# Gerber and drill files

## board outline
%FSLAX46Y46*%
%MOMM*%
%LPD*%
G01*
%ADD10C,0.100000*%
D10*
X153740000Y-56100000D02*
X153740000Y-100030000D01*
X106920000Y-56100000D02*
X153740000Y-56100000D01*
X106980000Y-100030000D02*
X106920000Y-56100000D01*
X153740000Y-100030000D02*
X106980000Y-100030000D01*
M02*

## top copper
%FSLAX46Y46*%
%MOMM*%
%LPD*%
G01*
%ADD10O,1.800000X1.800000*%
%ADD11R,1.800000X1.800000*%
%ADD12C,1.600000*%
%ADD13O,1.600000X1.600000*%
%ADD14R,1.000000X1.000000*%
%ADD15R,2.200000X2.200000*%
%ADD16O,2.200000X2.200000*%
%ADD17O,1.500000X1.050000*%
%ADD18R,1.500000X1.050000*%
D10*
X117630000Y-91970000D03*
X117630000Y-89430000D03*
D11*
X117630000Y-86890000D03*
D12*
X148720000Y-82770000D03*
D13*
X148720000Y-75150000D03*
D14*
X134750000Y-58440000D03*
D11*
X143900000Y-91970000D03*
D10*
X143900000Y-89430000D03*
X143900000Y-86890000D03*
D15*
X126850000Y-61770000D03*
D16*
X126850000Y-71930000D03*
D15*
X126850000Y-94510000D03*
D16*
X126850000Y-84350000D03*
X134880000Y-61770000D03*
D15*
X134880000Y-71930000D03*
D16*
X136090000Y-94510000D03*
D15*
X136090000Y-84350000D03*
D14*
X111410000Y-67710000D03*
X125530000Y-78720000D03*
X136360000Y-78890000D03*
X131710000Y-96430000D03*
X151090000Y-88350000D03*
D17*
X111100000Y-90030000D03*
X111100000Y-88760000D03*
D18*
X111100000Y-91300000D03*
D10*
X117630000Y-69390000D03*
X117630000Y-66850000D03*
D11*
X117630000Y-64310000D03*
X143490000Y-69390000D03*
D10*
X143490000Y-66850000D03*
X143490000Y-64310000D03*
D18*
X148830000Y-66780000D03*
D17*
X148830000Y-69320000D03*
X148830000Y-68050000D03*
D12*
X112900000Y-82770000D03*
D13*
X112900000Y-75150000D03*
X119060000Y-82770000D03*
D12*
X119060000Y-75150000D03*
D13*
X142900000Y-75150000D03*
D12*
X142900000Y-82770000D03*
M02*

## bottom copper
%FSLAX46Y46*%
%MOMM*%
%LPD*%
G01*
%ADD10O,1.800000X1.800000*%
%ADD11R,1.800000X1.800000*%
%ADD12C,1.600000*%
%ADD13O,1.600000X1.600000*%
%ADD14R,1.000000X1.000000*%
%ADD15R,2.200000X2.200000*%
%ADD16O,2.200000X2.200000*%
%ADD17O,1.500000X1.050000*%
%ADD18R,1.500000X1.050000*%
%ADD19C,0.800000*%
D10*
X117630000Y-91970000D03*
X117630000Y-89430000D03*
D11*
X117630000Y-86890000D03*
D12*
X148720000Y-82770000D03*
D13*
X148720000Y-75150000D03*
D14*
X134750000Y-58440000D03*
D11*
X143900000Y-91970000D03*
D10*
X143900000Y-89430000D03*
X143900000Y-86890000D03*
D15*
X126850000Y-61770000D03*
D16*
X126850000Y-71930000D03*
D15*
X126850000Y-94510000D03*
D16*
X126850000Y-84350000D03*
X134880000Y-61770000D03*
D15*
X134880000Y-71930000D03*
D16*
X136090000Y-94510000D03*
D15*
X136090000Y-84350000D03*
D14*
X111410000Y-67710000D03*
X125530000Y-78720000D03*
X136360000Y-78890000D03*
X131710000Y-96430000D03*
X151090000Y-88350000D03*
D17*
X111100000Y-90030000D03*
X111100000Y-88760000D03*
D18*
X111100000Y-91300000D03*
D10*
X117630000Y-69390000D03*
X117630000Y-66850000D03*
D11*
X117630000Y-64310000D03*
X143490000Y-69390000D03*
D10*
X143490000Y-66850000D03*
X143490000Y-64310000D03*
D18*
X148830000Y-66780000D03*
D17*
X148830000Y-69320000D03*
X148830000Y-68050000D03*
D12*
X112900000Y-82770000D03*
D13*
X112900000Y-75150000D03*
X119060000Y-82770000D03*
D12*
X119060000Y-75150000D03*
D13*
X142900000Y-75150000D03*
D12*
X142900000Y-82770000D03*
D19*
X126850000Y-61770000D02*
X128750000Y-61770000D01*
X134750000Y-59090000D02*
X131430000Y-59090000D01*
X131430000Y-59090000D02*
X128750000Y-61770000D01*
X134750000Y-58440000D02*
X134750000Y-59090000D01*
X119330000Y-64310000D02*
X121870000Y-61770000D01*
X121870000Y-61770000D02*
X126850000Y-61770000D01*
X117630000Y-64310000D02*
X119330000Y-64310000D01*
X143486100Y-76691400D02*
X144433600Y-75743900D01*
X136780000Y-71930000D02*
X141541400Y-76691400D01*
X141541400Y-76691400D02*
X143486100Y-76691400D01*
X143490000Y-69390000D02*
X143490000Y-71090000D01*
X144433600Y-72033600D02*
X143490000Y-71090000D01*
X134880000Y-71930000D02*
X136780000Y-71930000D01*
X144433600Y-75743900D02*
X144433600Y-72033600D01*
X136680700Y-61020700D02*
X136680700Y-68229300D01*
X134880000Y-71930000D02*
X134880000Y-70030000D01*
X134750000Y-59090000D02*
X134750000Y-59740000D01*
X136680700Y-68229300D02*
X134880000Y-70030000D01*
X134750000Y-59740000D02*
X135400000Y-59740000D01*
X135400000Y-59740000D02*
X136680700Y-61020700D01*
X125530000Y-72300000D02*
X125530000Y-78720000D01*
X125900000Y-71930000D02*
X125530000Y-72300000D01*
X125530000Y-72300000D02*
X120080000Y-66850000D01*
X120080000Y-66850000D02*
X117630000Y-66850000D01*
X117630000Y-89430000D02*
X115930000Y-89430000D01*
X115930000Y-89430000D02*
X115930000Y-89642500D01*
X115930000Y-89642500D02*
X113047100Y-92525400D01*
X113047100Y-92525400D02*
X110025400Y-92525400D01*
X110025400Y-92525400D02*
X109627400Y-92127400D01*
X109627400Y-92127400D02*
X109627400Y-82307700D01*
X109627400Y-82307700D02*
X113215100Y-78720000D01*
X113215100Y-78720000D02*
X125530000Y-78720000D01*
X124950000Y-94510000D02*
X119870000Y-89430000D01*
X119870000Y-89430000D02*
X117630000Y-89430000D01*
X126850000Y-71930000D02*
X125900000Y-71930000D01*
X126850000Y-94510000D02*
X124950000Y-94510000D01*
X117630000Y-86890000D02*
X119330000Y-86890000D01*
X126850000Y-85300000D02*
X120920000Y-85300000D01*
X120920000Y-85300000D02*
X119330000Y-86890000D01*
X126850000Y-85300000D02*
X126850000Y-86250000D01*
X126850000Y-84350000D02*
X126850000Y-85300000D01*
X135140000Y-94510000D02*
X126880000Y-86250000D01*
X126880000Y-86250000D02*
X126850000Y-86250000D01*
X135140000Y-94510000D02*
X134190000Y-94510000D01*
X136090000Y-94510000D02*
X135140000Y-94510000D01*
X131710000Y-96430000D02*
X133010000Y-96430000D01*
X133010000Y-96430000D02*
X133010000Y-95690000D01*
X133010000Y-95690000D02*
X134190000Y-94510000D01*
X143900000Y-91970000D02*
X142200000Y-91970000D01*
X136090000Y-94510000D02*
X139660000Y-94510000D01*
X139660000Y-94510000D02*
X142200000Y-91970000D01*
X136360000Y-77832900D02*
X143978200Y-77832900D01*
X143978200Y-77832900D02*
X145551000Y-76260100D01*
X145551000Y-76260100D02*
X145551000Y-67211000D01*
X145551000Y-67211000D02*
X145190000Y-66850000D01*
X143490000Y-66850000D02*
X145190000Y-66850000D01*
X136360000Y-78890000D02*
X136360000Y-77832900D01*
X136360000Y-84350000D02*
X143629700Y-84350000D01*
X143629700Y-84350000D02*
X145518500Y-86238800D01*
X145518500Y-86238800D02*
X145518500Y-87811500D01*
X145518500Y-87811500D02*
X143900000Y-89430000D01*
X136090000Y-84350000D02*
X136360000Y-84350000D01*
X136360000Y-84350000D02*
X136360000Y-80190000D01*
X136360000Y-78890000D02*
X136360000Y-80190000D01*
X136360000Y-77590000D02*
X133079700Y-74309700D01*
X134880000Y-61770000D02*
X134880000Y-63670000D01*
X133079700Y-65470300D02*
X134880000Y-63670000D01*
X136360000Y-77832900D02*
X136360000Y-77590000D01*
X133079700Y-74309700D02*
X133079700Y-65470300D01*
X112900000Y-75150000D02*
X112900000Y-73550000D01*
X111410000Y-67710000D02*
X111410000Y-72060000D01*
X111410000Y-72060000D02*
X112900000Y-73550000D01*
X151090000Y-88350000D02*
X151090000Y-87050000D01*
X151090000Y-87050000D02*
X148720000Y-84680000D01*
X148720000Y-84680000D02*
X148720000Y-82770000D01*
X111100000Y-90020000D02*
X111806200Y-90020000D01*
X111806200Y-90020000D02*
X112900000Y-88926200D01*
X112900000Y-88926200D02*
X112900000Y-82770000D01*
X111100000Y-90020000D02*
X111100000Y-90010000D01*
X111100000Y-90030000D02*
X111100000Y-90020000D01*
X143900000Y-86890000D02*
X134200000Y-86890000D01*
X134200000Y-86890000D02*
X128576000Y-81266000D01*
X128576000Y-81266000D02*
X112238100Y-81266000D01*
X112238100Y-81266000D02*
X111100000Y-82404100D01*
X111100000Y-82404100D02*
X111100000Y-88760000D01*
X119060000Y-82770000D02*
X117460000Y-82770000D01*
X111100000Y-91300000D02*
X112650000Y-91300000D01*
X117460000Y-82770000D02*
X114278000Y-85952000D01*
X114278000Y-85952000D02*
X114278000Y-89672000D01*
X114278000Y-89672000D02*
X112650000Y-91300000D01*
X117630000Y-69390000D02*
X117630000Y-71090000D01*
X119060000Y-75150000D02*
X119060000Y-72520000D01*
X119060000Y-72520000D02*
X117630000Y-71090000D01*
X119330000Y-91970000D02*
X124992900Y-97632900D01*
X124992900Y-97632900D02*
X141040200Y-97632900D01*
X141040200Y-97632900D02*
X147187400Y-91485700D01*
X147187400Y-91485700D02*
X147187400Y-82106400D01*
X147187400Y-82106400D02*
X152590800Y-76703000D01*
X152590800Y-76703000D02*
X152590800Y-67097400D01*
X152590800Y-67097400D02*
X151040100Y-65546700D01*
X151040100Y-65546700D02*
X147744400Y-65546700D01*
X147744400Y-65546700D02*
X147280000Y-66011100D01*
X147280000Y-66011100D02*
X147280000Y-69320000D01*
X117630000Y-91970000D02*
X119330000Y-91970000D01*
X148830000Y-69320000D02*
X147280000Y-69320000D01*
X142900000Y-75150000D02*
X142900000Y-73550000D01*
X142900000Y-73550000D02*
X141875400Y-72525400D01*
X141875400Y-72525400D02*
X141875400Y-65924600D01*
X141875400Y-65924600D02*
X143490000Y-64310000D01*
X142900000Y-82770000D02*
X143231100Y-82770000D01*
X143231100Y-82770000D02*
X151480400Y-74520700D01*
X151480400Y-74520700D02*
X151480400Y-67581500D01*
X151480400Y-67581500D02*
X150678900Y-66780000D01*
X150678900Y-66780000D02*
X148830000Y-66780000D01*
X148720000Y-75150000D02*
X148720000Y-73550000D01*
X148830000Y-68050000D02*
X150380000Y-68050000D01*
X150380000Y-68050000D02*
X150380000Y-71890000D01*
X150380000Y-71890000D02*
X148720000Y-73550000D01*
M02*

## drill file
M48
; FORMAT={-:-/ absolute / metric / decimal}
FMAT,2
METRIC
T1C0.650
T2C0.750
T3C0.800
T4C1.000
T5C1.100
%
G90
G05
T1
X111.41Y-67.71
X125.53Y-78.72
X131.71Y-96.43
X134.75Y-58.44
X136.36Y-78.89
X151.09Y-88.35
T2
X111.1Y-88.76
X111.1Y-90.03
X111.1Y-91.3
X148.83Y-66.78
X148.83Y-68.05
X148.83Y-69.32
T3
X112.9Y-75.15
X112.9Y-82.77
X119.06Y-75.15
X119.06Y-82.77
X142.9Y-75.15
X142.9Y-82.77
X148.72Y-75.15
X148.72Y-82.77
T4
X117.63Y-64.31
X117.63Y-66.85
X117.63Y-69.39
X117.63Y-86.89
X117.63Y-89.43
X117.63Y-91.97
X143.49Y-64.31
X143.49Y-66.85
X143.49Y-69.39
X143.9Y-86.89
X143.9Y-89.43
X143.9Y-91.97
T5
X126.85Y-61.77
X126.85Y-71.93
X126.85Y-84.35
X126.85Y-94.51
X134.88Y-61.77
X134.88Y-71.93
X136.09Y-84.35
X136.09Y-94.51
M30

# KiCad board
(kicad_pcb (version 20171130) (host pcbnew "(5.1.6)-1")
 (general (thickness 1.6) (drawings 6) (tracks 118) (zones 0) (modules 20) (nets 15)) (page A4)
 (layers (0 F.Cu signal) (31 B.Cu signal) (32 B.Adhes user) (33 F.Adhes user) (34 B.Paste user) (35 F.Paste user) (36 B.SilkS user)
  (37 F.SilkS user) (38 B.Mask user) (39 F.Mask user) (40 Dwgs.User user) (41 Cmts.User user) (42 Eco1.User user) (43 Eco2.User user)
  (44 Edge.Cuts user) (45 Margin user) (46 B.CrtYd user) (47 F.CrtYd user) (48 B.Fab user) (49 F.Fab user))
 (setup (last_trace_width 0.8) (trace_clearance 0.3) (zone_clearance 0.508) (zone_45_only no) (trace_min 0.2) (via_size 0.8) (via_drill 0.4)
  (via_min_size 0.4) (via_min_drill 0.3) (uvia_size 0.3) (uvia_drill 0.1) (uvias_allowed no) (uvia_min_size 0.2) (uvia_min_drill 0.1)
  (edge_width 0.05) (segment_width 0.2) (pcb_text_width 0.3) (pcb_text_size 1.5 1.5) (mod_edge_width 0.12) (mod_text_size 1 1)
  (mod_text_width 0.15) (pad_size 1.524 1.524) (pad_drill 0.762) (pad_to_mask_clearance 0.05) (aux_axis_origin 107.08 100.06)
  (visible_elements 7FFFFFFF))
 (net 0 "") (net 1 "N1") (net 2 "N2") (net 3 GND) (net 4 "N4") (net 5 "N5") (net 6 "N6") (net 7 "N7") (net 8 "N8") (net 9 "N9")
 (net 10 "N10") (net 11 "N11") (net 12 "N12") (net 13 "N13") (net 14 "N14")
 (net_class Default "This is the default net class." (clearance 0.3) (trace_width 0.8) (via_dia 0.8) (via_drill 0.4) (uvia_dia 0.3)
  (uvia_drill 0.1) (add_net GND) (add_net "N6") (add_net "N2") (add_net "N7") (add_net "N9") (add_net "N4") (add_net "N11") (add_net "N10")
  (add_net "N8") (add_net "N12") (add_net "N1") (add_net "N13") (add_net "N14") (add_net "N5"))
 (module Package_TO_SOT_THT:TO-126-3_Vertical (layer F.Cu) (at 117.63 86.89 270)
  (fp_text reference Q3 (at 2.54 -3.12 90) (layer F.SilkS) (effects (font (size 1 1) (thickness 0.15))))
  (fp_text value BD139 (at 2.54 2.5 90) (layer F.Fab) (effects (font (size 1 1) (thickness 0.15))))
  (pad 3 thru_hole oval (at 5.08 0 270) (size 1.8 1.8) (drill 1) (layers *.Cu *.Mask) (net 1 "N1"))
  (pad 2 thru_hole oval (at 2.54 0 270) (size 1.8 1.8) (drill 1) (layers *.Cu *.Mask) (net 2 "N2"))
  (pad 1 thru_hole rect (at 0 0 270) (size 1.8 1.8) (drill 1) (layers *.Cu *.Mask) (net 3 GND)))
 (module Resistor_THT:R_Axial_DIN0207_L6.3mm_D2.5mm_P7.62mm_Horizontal (layer F.Cu) (at 148.72 82.77 90)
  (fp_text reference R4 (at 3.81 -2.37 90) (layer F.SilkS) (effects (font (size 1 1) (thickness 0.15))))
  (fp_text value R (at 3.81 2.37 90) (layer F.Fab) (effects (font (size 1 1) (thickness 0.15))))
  (pad 1 thru_hole circle (at 0 0 90) (size 1.6 1.6) (drill 0.8) (layers *.Cu *.Mask) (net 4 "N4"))
  (pad 2 thru_hole oval (at 7.62 0 90) (size 1.6 1.6) (drill 0.8) (layers *.Cu *.Mask) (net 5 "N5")))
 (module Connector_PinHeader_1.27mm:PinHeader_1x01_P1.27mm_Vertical (layer F.Cu) (at 134.75 58.44)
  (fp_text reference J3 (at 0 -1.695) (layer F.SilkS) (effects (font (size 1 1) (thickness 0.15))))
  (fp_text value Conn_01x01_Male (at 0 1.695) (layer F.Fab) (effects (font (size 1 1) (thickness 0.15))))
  (pad 1 thru_hole rect (at 0 0) (size 1 1) (drill 0.65) (layers *.Cu *.Mask) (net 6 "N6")))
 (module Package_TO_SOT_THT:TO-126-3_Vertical (layer F.Cu) (at 143.9 91.97 90)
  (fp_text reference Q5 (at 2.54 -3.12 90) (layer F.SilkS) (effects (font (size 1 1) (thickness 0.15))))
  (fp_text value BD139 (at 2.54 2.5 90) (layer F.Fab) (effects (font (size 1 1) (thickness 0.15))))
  (pad 1 thru_hole rect (at 0 0 90) (size 1.8 1.8) (drill 1) (layers *.Cu *.Mask) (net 3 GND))
  (pad 2 thru_hole oval (at 2.54 0 90) (size 1.8 1.8) (drill 1) (layers *.Cu *.Mask) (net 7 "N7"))
  (pad 3 thru_hole oval (at 5.08 0 90) (size 1.8 1.8) (drill 1) (layers *.Cu *.Mask) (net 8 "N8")))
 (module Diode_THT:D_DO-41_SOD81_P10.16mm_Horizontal (layer F.Cu) (at 126.85 61.77 270)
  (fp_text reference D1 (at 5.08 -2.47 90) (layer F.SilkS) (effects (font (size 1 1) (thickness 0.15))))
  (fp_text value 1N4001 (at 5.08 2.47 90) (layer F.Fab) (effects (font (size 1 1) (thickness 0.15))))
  (pad 1 thru_hole rect (at 0 0 270) (size 2.2 2.2) (drill 1.1) (layers *.Cu *.Mask) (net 6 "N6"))
  (pad 2 thru_hole oval (at 10.16 0 270) (size 2.2 2.2) (drill 1.1) (layers *.Cu *.Mask) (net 2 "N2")))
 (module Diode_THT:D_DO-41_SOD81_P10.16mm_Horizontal (layer F.Cu) (at 126.85 94.51 90)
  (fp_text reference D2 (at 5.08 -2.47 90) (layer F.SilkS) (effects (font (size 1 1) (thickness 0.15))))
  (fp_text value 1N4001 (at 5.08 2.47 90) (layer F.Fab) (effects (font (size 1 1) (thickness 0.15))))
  (pad 1 thru_hole rect (at 0 0 90) (size 2.2 2.2) (drill 1.1) (layers *.Cu *.Mask) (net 2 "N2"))
  (pad 2 thru_hole oval (at 10.16 0 90) (size 2.2 2.2) (drill 1.1) (layers *.Cu *.Mask) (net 3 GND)))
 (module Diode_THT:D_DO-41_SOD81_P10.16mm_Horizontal (layer F.Cu) (at 134.88 71.93 90)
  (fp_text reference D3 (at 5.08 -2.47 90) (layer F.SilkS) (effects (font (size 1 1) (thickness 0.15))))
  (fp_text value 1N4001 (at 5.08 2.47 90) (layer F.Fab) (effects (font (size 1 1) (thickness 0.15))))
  (pad 2 thru_hole oval (at 10.16 0 90) (size 2.2 2.2) (drill 1.1) (layers *.Cu *.Mask) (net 7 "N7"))
  (pad 1 thru_hole rect (at 0 0 90) (size 2.2 2.2) (drill 1.1) (layers *.Cu *.Mask) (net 6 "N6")))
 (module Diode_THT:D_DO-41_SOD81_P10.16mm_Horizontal (layer F.Cu) (at 136.09 84.35 270)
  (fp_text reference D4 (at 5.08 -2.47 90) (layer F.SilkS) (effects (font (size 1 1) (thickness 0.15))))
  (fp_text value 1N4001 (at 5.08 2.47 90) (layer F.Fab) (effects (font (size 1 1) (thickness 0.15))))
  (pad 2 thru_hole oval (at 10.16 0 270) (size 2.2 2.2) (drill 1.1) (layers *.Cu *.Mask) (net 3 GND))
  (pad 1 thru_hole rect (at 0 0 270) (size 2.2 2.2) (drill 1.1) (layers *.Cu *.Mask) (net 7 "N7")))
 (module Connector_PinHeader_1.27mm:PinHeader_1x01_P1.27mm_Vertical (layer F.Cu) (at 111.41 67.71)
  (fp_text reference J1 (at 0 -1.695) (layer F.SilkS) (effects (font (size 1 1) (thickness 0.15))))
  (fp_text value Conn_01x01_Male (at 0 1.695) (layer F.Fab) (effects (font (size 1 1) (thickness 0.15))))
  (pad 1 thru_hole rect (at 0 0) (size 1 1) (drill 0.65) (layers *.Cu *.Mask) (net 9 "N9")))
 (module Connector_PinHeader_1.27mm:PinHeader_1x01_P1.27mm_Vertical (layer F.Cu) (at 125.53 78.72)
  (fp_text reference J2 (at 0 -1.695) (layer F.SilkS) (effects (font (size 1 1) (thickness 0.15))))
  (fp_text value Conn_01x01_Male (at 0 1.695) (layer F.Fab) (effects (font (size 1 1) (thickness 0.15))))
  (pad 1 thru_hole rect (at 0 0) (size 1 1) (drill 0.65) (layers *.Cu *.Mask) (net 2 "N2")))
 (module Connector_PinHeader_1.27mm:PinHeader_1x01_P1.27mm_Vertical (layer F.Cu) (at 136.36 78.89)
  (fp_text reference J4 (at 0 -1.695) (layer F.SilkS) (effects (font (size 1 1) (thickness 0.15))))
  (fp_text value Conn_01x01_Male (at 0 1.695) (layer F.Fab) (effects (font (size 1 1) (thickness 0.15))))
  (pad 1 thru_hole rect (at 0 0) (size 1 1) (drill 0.65) (layers *.Cu *.Mask) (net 7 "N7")))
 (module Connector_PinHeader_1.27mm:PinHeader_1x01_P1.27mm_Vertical (layer F.Cu) (at 131.71 96.43)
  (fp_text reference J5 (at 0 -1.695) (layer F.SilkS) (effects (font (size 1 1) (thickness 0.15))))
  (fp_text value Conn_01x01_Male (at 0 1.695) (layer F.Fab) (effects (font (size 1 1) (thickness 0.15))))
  (pad 1 thru_hole rect (at 0 0) (size 1 1) (drill 0.65) (layers *.Cu *.Mask) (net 3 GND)))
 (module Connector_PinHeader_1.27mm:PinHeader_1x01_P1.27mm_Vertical (layer F.Cu) (at 151.09 88.35)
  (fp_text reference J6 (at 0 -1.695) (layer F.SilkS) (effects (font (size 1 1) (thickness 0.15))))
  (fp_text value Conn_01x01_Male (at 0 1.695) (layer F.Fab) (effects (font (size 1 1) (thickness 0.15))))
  (pad 1 thru_hole rect (at 0 0) (size 1 1) (drill 0.65) (layers *.Cu *.Mask) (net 4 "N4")))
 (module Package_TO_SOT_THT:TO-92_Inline (layer F.Cu) (at 111.1 91.3 90)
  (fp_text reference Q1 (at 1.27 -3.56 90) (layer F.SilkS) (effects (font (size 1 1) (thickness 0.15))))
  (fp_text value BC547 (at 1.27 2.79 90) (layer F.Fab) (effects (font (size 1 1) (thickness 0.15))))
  (pad 2 thru_hole oval (at 1.27 0 90) (size 1.05 1.5) (drill 0.75) (layers *.Cu *.Mask) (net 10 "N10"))
  (pad 3 thru_hole oval (at 2.54 0 90) (size 1.05 1.5) (drill 0.75) (layers *.Cu *.Mask) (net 8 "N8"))
  (pad 1 thru_hole rect (at 0 0 90) (size 1.05 1.5) (drill 0.75) (layers *.Cu *.Mask) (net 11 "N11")))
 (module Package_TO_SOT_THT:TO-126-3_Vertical (layer F.Cu) (at 117.63 64.31 270)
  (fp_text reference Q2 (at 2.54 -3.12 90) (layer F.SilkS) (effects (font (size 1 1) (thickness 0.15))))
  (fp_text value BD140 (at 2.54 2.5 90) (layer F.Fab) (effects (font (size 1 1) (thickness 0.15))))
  (pad 3 thru_hole oval (at 5.08 0 270) (size 1.8 1.8) (drill 1) (layers *.Cu *.Mask) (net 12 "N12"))
  (pad 2 thru_hole oval (at 2.54 0 270) (size 1.8 1.8) (drill 1) (layers *.Cu *.Mask) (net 2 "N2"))
  (pad 1 thru_hole rect (at 0 0 270) (size 1.8 1.8) (drill 1) (layers *.Cu *.Mask) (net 6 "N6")))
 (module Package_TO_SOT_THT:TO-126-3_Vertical (layer F.Cu) (at 143.49 69.39 90)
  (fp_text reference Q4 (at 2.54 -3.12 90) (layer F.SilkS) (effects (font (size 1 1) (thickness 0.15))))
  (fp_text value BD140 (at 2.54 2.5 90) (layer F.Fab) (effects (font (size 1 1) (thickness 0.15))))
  (pad 1 thru_hole rect (at 0 0 90) (size 1.8 1.8) (drill 1) (layers *.Cu *.Mask) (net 6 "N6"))
  (pad 2 thru_hole oval (at 2.54 0 90) (size 1.8 1.8) (drill 1) (layers *.Cu *.Mask) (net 7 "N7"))
  (pad 3 thru_hole oval (at 5.08 0 90) (size 1.8 1.8) (drill 1) (layers *.Cu *.Mask) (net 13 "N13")))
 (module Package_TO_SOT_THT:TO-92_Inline (layer F.Cu) (at 148.83 66.78 270)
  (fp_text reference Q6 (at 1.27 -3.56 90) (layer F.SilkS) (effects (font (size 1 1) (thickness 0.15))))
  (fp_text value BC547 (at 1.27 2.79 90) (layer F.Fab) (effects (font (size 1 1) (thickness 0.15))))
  (pad 1 thru_hole rect (at 0 0 270) (size 1.05 1.5) (drill 0.75) (layers *.Cu *.Mask) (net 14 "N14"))
  (pad 3 thru_hole oval (at 2.54 0 270) (size 1.05 1.5) (drill 0.75) (layers *.Cu *.Mask) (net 1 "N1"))
  (pad 2 thru_hole oval (at 1.27 0 270) (size 1.05 1.5) (drill 0.75) (layers *.Cu *.Mask) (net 5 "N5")))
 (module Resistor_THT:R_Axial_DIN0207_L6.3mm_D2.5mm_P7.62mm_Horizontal (layer F.Cu) (at 112.9 82.77 90)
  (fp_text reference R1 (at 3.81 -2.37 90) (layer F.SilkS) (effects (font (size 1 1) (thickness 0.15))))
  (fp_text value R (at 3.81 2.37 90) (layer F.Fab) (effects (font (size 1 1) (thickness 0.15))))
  (pad 1 thru_hole circle (at 0 0 90) (size 1.6 1.6) (drill 0.8) (layers *.Cu *.Mask) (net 10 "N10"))
  (pad 2 thru_hole oval (at 7.62 0 90) (size 1.6 1.6) (drill 0.8) (layers *.Cu *.Mask) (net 9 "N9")))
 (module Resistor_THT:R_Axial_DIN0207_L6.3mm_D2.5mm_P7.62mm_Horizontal (layer F.Cu) (at 119.06 75.15 270)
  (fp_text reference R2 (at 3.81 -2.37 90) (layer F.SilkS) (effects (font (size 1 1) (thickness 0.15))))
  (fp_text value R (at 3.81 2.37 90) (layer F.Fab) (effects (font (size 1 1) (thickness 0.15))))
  (pad 2 thru_hole oval (at 7.62 0 270) (size 1.6 1.6) (drill 0.8) (layers *.Cu *.Mask) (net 11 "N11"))
  (pad 1 thru_hole circle (at 0 0 270) (size 1.6 1.6) (drill 0.8) (layers *.Cu *.Mask) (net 12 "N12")))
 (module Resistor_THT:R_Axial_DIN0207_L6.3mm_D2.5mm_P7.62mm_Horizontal (layer F.Cu) (at 142.9 82.77 90)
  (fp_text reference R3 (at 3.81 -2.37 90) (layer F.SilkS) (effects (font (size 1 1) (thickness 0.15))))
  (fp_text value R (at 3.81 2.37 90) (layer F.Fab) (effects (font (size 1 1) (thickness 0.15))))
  (pad 2 thru_hole oval (at 7.62 0 90) (size 1.6 1.6) (drill 0.8) (layers *.Cu *.Mask) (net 13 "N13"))
  (pad 1 thru_hole circle (at 0 0 90) (size 1.6 1.6) (drill 0.8) (layers *.Cu *.Mask) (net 14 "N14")))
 (gr_line (start 153.74 56.1) (end 153.74 100.03) (layer Edge.Cuts) (width 0.1))
 (gr_line (start 106.92 56.1) (end 153.74 56.1) (layer Edge.Cuts) (width 0.1))
 (gr_line (start 106.98 100.03) (end 106.92 56.1) (layer Edge.Cuts) (width 0.1))
 (gr_line (start 153.74 100.03) (end 106.98 100.03) (layer Edge.Cuts) (width 0.1))
 (segment (start 126.85 61.77) (end 128.75 61.77) (width 0.8) (layer B.Cu) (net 6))
 (segment (start 134.75 59.09) (end 131.43 59.09) (width 0.8) (layer B.Cu) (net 6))
 (segment (start 131.43 59.09) (end 128.75 61.77) (width 0.8) (layer B.Cu) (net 6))
 (segment (start 134.75 58.44) (end 134.75 59.09) (width 0.8) (layer B.Cu) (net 6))
 (segment (start 119.33 64.31) (end 121.87 61.77) (width 0.8) (layer B.Cu) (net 6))
 (segment (start 121.87 61.77) (end 126.85 61.77) (width 0.8) (layer B.Cu) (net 6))
 (segment (start 117.63 64.31) (end 119.33 64.31) (width 0.8) (layer B.Cu) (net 6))
 (segment (start 143.4861 76.6914) (end 144.4336 75.7439) (width 0.8) (layer B.Cu) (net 6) (status 1000000))
 (segment (start 136.78 71.93) (end 141.5414 76.6914) (width 0.8) (layer B.Cu) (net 6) (status 1000000))
 (segment (start 141.5414 76.6914) (end 143.4861 76.6914) (width 0.8) (layer B.Cu) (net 6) (status 1000000))
 (segment (start 143.49 69.39) (end 143.49 71.09) (width 0.8) (layer B.Cu) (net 6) (status 1000000))
 (segment (start 144.4336 72.0336) (end 143.49 71.09) (width 0.8) (layer B.Cu) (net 6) (status 1000000))
 (segment (start 134.88 71.93) (end 136.78 71.93) (width 0.8) (layer B.Cu) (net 6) (status 1000000))
 (segment (start 144.4336 75.7439) (end 144.4336 72.0336) (width 0.8) (layer B.Cu) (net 6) (status 1000000))
 (segment (start 136.6807 61.0207) (end 136.6807 68.2293) (width 0.8) (layer B.Cu) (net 6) (status 1000000))
 (segment (start 134.88 71.93) (end 134.88 70.03) (width 0.8) (layer B.Cu) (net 6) (status 1000000))
 (segment (start 134.75 59.09) (end 134.75 59.74) (width 0.8) (layer B.Cu) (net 6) (status 1000000))
 (segment (start 136.6807 68.2293) (end 134.88 70.03) (width 0.8) (layer B.Cu) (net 6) (status 1000000))
 (segment (start 134.75 59.74) (end 135.4 59.74) (width 0.8) (layer B.Cu) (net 6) (status 1000000))
 (segment (start 135.4 59.74) (end 136.6807 61.0207) (width 0.8) (layer B.Cu) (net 6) (status 1000000))
 (segment (start 125.53 72.3) (end 125.53 78.72) (width 0.8) (layer B.Cu) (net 2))
 (segment (start 125.9 71.93) (end 125.53 72.3) (width 0.8) (layer B.Cu) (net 2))
 (segment (start 125.53 72.3) (end 120.08 66.85) (width 0.8) (layer B.Cu) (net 2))
 (segment (start 120.08 66.85) (end 117.63 66.85) (width 0.8) (layer B.Cu) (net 2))
 (segment (start 117.63 89.43) (end 115.93 89.43) (width 0.8) (layer B.Cu) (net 2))
 (segment (start 115.93 89.43) (end 115.93 89.6425) (width 0.8) (layer B.Cu) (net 2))
 (segment (start 115.93 89.6425) (end 113.0471 92.5254) (width 0.8) (layer B.Cu) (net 2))
 (segment (start 113.0471 92.5254) (end 110.0254 92.5254) (width 0.8) (layer B.Cu) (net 2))
 (segment (start 110.0254 92.5254) (end 109.6274 92.1274) (width 0.8) (layer B.Cu) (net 2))
 (segment (start 109.6274 92.1274) (end 109.6274 82.3077) (width 0.8) (layer B.Cu) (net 2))
 (segment (start 109.6274 82.3077) (end 113.2151 78.72) (width 0.8) (layer B.Cu) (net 2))
 (segment (start 113.2151 78.72) (end 125.53 78.72) (width 0.8) (layer B.Cu) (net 2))
 (segment (start 124.95 94.51) (end 119.87 89.43) (width 0.8) (layer B.Cu) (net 2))
 (segment (start 119.87 89.43) (end 117.63 89.43) (width 0.8) (layer B.Cu) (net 2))
 (segment (start 126.85 71.93) (end 125.9 71.93) (width 0.8) (layer B.Cu) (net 2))
 (segment (start 126.85 94.51) (end 124.95 94.51) (width 0.8) (layer B.Cu) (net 2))
 (segment (start 117.63 86.89) (end 119.33 86.89) (width 0.8) (layer B.Cu) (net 3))
 (segment (start 126.85 85.3) (end 120.92 85.3) (width 0.8) (layer B.Cu) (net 3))
 (segment (start 120.92 85.3) (end 119.33 86.89) (width 0.8) (layer B.Cu) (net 3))
 (segment (start 126.85 85.3) (end 126.85 86.25) (width 0.8) (layer B.Cu) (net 3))
 (segment (start 126.85 84.35) (end 126.85 85.3) (width 0.8) (layer B.Cu) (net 3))
 (segment (start 135.14 94.51) (end 126.88 86.25) (width 0.8) (layer B.Cu) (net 3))
 (segment (start 126.88 86.25) (end 126.85 86.25) (width 0.8) (layer B.Cu) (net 3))
 (segment (start 135.14 94.51) (end 134.19 94.51) (width 0.8) (layer B.Cu) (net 3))
 (segment (start 136.09 94.51) (end 135.14 94.51) (width 0.8) (layer B.Cu) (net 3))
 (segment (start 131.71 96.43) (end 133.01 96.43) (width 0.8) (layer B.Cu) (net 3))
 (segment (start 133.01 96.43) (end 133.01 95.69) (width 0.8) (layer B.Cu) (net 3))
 (segment (start 133.01 95.69) (end 134.19 94.51) (width 0.8) (layer B.Cu) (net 3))
 (segment (start 143.9 91.97) (end 142.2 91.97) (width 0.8) (layer B.Cu) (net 3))
 (segment (start 136.09 94.51) (end 139.66 94.51) (width 0.8) (layer B.Cu) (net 3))
 (segment (start 139.66 94.51) (end 142.2 91.97) (width 0.8) (layer B.Cu) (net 3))
 (segment (start 136.36 77.8329) (end 143.9782 77.8329) (width 0.8) (layer B.Cu) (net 7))
 (segment (start 143.9782 77.8329) (end 145.551 76.2601) (width 0.8) (layer B.Cu) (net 7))
 (segment (start 145.551 76.2601) (end 145.551 67.211) (width 0.8) (layer B.Cu) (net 7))
 (segment (start 145.551 67.211) (end 145.19 66.85) (width 0.8) (layer B.Cu) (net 7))
 (segment (start 143.49 66.85) (end 145.19 66.85) (width 0.8) (layer B.Cu) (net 7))
 (segment (start 136.36 78.89) (end 136.36 77.8329) (width 0.8) (layer B.Cu) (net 7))
 (segment (start 136.36 84.35) (end 143.6297 84.35) (width 0.8) (layer B.Cu) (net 7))
 (segment (start 143.6297 84.35) (end 145.5185 86.2388) (width 0.8) (layer B.Cu) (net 7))
 (segment (start 145.5185 86.2388) (end 145.5185 87.8115) (width 0.8) (layer B.Cu) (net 7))
 (segment (start 145.5185 87.8115) (end 143.9 89.43) (width 0.8) (layer B.Cu) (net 7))
 (segment (start 136.09 84.35) (end 136.36 84.35) (width 0.8) (layer B.Cu) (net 7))
 (segment (start 136.36 84.35) (end 136.36 80.19) (width 0.8) (layer B.Cu) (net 7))
 (segment (start 136.36 78.89) (end 136.36 80.19) (width 0.8) (layer B.Cu) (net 7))
 (segment (start 136.36 77.59) (end 133.0797 74.3097) (width 0.8) (layer B.Cu) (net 7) (status 1000000))
 (segment (start 134.88 61.77) (end 134.88 63.67) (width 0.8) (layer B.Cu) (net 7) (status 1000000))
 (segment (start 133.0797 65.4703) (end 134.88 63.67) (width 0.8) (layer B.Cu) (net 7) (status 1000000))
 (segment (start 136.36 77.8329) (end 136.36 77.59) (width 0.8) (layer B.Cu) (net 7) (status 1000000))
 (segment (start 133.0797 74.3097) (end 133.0797 65.4703) (width 0.8) (layer B.Cu) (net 7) (status 1000000))
 (segment (start 112.9 75.15) (end 112.9 73.55) (width 0.8) (layer B.Cu) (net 9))
 (segment (start 111.41 67.71) (end 111.41 72.06) (width 0.8) (layer B.Cu) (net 9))
 (segment (start 111.41 72.06) (end 112.9 73.55) (width 0.8) (layer B.Cu) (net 9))
 (segment (start 151.09 88.35) (end 151.09 87.05) (width 0.8) (layer B.Cu) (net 4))
 (segment (start 151.09 87.05) (end 148.72 84.68) (width 0.8) (layer B.Cu) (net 4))
 (segment (start 148.72 84.68) (end 148.72 82.77) (width 0.8) (layer B.Cu) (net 4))
 (segment (start 111.1 90.02) (end 111.8062 90.02) (width 0.8) (layer B.Cu) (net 10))
 (segment (start 111.8062 90.02) (end 112.9 88.9262) (width 0.8) (layer B.Cu) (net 10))
 (segment (start 112.9 88.9262) (end 112.9 82.77) (width 0.8) (layer B.Cu) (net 10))
 (segment (start 111.1 90.02) (end 111.1 90.01) (width 0.8) (layer B.Cu) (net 10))
 (segment (start 111.1 90.03) (end 111.1 90.02) (width 0.8) (layer B.Cu) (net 10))
 (segment (start 143.9 86.89) (end 134.2 86.89) (width 0.8) (layer B.Cu) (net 8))
 (segment (start 134.2 86.89) (end 128.576 81.266) (width 0.8) (layer B.Cu) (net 8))
 (segment (start 128.576 81.266) (end 112.2381 81.266) (width 0.8) (layer B.Cu) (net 8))
 (segment (start 112.2381 81.266) (end 111.1 82.4041) (width 0.8) (layer B.Cu) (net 8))
 (segment (start 111.1 82.4041) (end 111.1 88.76) (width 0.8) (layer B.Cu) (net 8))
 (segment (start 119.06 82.77) (end 117.46 82.77) (width 0.8) (layer B.Cu) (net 11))
 (segment (start 111.1 91.3) (end 112.65 91.3) (width 0.8) (layer B.Cu) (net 11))
 (segment (start 117.46 82.77) (end 114.278 85.952) (width 0.8) (layer B.Cu) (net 11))
 (segment (start 114.278 85.952) (end 114.278 89.672) (width 0.8) (layer B.Cu) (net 11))
 (segment (start 114.278 89.672) (end 112.65 91.3) (width 0.8) (layer B.Cu) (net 11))
 (segment (start 117.63 69.39) (end 117.63 71.09) (width 0.8) (layer B.Cu) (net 12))
 (segment (start 119.06 75.15) (end 119.06 72.52) (width 0.8) (layer B.Cu) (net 12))
 (segment (start 119.06 72.52) (end 117.63 71.09) (width 0.8) (layer B.Cu) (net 12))
 (segment (start 119.33 91.97) (end 124.9929 97.6329) (width 0.8) (layer B.Cu) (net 1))
 (segment (start 124.9929 97.6329) (end 141.0402 97.6329) (width 0.8) (layer B.Cu) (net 1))
 (segment (start 141.0402 97.6329) (end 147.1874 91.4857) (width 0.8) (layer B.Cu) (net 1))
 (segment (start 147.1874 91.4857) (end 147.1874 82.1064) (width 0.8) (layer B.Cu) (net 1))
 (segment (start 147.1874 82.1064) (end 152.5908 76.703) (width 0.8) (layer B.Cu) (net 1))
 (segment (start 152.5908 76.703) (end 152.5908 67.0974) (width 0.8) (layer B.Cu) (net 1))
 (segment (start 152.5908 67.0974) (end 151.0401 65.5467) (width 0.8) (layer B.Cu) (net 1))
 (segment (start 151.0401 65.5467) (end 147.7444 65.5467) (width 0.8) (layer B.Cu) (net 1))
 (segment (start 147.7444 65.5467) (end 147.28 66.0111) (width 0.8) (layer B.Cu) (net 1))
 (segment (start 147.28 66.0111) (end 147.28 69.32) (width 0.8) (layer B.Cu) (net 1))
 (segment (start 117.63 91.97) (end 119.33 91.97) (width 0.8) (layer B.Cu) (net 1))
 (segment (start 148.83 69.32) (end 147.28 69.32) (width 0.8) (layer B.Cu) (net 1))
 (segment (start 142.9 75.15) (end 142.9 73.55) (width 0.8) (layer B.Cu) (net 13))
 (segment (start 142.9 73.55) (end 141.8754 72.5254) (width 0.8) (layer B.Cu) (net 13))
 (segment (start 141.8754 72.5254) (end 141.8754 65.9246) (width 0.8) (layer B.Cu) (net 13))
 (segment (start 141.8754 65.9246) (end 143.49 64.31) (width 0.8) (layer B.Cu) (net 13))
 (segment (start 142.9 82.77) (end 143.2311 82.77) (width 0.8) (layer B.Cu) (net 14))
 (segment (start 143.2311 82.77) (end 151.4804 74.5207) (width 0.8) (layer B.Cu) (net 14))
 (segment (start 151.4804 74.5207) (end 151.4804 67.5815) (width 0.8) (layer B.Cu) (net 14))
 (segment (start 151.4804 67.5815) (end 150.6789 66.78) (width 0.8) (layer B.Cu) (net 14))
 (segment (start 150.6789 66.78) (end 148.83 66.78) (width 0.8) (layer B.Cu) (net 14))
 (segment (start 148.72 75.15) (end 148.72 73.55) (width 0.8) (layer B.Cu) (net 5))
 (segment (start 148.83 68.05) (end 150.38 68.05) (width 0.8) (layer B.Cu) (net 5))
 (segment (start 150.38 68.05) (end 150.38 71.89) (width 0.8) (layer B.Cu) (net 5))
 (segment (start 150.38 71.89) (end 148.72 73.55) (width 0.8) (layer B.Cu) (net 5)))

